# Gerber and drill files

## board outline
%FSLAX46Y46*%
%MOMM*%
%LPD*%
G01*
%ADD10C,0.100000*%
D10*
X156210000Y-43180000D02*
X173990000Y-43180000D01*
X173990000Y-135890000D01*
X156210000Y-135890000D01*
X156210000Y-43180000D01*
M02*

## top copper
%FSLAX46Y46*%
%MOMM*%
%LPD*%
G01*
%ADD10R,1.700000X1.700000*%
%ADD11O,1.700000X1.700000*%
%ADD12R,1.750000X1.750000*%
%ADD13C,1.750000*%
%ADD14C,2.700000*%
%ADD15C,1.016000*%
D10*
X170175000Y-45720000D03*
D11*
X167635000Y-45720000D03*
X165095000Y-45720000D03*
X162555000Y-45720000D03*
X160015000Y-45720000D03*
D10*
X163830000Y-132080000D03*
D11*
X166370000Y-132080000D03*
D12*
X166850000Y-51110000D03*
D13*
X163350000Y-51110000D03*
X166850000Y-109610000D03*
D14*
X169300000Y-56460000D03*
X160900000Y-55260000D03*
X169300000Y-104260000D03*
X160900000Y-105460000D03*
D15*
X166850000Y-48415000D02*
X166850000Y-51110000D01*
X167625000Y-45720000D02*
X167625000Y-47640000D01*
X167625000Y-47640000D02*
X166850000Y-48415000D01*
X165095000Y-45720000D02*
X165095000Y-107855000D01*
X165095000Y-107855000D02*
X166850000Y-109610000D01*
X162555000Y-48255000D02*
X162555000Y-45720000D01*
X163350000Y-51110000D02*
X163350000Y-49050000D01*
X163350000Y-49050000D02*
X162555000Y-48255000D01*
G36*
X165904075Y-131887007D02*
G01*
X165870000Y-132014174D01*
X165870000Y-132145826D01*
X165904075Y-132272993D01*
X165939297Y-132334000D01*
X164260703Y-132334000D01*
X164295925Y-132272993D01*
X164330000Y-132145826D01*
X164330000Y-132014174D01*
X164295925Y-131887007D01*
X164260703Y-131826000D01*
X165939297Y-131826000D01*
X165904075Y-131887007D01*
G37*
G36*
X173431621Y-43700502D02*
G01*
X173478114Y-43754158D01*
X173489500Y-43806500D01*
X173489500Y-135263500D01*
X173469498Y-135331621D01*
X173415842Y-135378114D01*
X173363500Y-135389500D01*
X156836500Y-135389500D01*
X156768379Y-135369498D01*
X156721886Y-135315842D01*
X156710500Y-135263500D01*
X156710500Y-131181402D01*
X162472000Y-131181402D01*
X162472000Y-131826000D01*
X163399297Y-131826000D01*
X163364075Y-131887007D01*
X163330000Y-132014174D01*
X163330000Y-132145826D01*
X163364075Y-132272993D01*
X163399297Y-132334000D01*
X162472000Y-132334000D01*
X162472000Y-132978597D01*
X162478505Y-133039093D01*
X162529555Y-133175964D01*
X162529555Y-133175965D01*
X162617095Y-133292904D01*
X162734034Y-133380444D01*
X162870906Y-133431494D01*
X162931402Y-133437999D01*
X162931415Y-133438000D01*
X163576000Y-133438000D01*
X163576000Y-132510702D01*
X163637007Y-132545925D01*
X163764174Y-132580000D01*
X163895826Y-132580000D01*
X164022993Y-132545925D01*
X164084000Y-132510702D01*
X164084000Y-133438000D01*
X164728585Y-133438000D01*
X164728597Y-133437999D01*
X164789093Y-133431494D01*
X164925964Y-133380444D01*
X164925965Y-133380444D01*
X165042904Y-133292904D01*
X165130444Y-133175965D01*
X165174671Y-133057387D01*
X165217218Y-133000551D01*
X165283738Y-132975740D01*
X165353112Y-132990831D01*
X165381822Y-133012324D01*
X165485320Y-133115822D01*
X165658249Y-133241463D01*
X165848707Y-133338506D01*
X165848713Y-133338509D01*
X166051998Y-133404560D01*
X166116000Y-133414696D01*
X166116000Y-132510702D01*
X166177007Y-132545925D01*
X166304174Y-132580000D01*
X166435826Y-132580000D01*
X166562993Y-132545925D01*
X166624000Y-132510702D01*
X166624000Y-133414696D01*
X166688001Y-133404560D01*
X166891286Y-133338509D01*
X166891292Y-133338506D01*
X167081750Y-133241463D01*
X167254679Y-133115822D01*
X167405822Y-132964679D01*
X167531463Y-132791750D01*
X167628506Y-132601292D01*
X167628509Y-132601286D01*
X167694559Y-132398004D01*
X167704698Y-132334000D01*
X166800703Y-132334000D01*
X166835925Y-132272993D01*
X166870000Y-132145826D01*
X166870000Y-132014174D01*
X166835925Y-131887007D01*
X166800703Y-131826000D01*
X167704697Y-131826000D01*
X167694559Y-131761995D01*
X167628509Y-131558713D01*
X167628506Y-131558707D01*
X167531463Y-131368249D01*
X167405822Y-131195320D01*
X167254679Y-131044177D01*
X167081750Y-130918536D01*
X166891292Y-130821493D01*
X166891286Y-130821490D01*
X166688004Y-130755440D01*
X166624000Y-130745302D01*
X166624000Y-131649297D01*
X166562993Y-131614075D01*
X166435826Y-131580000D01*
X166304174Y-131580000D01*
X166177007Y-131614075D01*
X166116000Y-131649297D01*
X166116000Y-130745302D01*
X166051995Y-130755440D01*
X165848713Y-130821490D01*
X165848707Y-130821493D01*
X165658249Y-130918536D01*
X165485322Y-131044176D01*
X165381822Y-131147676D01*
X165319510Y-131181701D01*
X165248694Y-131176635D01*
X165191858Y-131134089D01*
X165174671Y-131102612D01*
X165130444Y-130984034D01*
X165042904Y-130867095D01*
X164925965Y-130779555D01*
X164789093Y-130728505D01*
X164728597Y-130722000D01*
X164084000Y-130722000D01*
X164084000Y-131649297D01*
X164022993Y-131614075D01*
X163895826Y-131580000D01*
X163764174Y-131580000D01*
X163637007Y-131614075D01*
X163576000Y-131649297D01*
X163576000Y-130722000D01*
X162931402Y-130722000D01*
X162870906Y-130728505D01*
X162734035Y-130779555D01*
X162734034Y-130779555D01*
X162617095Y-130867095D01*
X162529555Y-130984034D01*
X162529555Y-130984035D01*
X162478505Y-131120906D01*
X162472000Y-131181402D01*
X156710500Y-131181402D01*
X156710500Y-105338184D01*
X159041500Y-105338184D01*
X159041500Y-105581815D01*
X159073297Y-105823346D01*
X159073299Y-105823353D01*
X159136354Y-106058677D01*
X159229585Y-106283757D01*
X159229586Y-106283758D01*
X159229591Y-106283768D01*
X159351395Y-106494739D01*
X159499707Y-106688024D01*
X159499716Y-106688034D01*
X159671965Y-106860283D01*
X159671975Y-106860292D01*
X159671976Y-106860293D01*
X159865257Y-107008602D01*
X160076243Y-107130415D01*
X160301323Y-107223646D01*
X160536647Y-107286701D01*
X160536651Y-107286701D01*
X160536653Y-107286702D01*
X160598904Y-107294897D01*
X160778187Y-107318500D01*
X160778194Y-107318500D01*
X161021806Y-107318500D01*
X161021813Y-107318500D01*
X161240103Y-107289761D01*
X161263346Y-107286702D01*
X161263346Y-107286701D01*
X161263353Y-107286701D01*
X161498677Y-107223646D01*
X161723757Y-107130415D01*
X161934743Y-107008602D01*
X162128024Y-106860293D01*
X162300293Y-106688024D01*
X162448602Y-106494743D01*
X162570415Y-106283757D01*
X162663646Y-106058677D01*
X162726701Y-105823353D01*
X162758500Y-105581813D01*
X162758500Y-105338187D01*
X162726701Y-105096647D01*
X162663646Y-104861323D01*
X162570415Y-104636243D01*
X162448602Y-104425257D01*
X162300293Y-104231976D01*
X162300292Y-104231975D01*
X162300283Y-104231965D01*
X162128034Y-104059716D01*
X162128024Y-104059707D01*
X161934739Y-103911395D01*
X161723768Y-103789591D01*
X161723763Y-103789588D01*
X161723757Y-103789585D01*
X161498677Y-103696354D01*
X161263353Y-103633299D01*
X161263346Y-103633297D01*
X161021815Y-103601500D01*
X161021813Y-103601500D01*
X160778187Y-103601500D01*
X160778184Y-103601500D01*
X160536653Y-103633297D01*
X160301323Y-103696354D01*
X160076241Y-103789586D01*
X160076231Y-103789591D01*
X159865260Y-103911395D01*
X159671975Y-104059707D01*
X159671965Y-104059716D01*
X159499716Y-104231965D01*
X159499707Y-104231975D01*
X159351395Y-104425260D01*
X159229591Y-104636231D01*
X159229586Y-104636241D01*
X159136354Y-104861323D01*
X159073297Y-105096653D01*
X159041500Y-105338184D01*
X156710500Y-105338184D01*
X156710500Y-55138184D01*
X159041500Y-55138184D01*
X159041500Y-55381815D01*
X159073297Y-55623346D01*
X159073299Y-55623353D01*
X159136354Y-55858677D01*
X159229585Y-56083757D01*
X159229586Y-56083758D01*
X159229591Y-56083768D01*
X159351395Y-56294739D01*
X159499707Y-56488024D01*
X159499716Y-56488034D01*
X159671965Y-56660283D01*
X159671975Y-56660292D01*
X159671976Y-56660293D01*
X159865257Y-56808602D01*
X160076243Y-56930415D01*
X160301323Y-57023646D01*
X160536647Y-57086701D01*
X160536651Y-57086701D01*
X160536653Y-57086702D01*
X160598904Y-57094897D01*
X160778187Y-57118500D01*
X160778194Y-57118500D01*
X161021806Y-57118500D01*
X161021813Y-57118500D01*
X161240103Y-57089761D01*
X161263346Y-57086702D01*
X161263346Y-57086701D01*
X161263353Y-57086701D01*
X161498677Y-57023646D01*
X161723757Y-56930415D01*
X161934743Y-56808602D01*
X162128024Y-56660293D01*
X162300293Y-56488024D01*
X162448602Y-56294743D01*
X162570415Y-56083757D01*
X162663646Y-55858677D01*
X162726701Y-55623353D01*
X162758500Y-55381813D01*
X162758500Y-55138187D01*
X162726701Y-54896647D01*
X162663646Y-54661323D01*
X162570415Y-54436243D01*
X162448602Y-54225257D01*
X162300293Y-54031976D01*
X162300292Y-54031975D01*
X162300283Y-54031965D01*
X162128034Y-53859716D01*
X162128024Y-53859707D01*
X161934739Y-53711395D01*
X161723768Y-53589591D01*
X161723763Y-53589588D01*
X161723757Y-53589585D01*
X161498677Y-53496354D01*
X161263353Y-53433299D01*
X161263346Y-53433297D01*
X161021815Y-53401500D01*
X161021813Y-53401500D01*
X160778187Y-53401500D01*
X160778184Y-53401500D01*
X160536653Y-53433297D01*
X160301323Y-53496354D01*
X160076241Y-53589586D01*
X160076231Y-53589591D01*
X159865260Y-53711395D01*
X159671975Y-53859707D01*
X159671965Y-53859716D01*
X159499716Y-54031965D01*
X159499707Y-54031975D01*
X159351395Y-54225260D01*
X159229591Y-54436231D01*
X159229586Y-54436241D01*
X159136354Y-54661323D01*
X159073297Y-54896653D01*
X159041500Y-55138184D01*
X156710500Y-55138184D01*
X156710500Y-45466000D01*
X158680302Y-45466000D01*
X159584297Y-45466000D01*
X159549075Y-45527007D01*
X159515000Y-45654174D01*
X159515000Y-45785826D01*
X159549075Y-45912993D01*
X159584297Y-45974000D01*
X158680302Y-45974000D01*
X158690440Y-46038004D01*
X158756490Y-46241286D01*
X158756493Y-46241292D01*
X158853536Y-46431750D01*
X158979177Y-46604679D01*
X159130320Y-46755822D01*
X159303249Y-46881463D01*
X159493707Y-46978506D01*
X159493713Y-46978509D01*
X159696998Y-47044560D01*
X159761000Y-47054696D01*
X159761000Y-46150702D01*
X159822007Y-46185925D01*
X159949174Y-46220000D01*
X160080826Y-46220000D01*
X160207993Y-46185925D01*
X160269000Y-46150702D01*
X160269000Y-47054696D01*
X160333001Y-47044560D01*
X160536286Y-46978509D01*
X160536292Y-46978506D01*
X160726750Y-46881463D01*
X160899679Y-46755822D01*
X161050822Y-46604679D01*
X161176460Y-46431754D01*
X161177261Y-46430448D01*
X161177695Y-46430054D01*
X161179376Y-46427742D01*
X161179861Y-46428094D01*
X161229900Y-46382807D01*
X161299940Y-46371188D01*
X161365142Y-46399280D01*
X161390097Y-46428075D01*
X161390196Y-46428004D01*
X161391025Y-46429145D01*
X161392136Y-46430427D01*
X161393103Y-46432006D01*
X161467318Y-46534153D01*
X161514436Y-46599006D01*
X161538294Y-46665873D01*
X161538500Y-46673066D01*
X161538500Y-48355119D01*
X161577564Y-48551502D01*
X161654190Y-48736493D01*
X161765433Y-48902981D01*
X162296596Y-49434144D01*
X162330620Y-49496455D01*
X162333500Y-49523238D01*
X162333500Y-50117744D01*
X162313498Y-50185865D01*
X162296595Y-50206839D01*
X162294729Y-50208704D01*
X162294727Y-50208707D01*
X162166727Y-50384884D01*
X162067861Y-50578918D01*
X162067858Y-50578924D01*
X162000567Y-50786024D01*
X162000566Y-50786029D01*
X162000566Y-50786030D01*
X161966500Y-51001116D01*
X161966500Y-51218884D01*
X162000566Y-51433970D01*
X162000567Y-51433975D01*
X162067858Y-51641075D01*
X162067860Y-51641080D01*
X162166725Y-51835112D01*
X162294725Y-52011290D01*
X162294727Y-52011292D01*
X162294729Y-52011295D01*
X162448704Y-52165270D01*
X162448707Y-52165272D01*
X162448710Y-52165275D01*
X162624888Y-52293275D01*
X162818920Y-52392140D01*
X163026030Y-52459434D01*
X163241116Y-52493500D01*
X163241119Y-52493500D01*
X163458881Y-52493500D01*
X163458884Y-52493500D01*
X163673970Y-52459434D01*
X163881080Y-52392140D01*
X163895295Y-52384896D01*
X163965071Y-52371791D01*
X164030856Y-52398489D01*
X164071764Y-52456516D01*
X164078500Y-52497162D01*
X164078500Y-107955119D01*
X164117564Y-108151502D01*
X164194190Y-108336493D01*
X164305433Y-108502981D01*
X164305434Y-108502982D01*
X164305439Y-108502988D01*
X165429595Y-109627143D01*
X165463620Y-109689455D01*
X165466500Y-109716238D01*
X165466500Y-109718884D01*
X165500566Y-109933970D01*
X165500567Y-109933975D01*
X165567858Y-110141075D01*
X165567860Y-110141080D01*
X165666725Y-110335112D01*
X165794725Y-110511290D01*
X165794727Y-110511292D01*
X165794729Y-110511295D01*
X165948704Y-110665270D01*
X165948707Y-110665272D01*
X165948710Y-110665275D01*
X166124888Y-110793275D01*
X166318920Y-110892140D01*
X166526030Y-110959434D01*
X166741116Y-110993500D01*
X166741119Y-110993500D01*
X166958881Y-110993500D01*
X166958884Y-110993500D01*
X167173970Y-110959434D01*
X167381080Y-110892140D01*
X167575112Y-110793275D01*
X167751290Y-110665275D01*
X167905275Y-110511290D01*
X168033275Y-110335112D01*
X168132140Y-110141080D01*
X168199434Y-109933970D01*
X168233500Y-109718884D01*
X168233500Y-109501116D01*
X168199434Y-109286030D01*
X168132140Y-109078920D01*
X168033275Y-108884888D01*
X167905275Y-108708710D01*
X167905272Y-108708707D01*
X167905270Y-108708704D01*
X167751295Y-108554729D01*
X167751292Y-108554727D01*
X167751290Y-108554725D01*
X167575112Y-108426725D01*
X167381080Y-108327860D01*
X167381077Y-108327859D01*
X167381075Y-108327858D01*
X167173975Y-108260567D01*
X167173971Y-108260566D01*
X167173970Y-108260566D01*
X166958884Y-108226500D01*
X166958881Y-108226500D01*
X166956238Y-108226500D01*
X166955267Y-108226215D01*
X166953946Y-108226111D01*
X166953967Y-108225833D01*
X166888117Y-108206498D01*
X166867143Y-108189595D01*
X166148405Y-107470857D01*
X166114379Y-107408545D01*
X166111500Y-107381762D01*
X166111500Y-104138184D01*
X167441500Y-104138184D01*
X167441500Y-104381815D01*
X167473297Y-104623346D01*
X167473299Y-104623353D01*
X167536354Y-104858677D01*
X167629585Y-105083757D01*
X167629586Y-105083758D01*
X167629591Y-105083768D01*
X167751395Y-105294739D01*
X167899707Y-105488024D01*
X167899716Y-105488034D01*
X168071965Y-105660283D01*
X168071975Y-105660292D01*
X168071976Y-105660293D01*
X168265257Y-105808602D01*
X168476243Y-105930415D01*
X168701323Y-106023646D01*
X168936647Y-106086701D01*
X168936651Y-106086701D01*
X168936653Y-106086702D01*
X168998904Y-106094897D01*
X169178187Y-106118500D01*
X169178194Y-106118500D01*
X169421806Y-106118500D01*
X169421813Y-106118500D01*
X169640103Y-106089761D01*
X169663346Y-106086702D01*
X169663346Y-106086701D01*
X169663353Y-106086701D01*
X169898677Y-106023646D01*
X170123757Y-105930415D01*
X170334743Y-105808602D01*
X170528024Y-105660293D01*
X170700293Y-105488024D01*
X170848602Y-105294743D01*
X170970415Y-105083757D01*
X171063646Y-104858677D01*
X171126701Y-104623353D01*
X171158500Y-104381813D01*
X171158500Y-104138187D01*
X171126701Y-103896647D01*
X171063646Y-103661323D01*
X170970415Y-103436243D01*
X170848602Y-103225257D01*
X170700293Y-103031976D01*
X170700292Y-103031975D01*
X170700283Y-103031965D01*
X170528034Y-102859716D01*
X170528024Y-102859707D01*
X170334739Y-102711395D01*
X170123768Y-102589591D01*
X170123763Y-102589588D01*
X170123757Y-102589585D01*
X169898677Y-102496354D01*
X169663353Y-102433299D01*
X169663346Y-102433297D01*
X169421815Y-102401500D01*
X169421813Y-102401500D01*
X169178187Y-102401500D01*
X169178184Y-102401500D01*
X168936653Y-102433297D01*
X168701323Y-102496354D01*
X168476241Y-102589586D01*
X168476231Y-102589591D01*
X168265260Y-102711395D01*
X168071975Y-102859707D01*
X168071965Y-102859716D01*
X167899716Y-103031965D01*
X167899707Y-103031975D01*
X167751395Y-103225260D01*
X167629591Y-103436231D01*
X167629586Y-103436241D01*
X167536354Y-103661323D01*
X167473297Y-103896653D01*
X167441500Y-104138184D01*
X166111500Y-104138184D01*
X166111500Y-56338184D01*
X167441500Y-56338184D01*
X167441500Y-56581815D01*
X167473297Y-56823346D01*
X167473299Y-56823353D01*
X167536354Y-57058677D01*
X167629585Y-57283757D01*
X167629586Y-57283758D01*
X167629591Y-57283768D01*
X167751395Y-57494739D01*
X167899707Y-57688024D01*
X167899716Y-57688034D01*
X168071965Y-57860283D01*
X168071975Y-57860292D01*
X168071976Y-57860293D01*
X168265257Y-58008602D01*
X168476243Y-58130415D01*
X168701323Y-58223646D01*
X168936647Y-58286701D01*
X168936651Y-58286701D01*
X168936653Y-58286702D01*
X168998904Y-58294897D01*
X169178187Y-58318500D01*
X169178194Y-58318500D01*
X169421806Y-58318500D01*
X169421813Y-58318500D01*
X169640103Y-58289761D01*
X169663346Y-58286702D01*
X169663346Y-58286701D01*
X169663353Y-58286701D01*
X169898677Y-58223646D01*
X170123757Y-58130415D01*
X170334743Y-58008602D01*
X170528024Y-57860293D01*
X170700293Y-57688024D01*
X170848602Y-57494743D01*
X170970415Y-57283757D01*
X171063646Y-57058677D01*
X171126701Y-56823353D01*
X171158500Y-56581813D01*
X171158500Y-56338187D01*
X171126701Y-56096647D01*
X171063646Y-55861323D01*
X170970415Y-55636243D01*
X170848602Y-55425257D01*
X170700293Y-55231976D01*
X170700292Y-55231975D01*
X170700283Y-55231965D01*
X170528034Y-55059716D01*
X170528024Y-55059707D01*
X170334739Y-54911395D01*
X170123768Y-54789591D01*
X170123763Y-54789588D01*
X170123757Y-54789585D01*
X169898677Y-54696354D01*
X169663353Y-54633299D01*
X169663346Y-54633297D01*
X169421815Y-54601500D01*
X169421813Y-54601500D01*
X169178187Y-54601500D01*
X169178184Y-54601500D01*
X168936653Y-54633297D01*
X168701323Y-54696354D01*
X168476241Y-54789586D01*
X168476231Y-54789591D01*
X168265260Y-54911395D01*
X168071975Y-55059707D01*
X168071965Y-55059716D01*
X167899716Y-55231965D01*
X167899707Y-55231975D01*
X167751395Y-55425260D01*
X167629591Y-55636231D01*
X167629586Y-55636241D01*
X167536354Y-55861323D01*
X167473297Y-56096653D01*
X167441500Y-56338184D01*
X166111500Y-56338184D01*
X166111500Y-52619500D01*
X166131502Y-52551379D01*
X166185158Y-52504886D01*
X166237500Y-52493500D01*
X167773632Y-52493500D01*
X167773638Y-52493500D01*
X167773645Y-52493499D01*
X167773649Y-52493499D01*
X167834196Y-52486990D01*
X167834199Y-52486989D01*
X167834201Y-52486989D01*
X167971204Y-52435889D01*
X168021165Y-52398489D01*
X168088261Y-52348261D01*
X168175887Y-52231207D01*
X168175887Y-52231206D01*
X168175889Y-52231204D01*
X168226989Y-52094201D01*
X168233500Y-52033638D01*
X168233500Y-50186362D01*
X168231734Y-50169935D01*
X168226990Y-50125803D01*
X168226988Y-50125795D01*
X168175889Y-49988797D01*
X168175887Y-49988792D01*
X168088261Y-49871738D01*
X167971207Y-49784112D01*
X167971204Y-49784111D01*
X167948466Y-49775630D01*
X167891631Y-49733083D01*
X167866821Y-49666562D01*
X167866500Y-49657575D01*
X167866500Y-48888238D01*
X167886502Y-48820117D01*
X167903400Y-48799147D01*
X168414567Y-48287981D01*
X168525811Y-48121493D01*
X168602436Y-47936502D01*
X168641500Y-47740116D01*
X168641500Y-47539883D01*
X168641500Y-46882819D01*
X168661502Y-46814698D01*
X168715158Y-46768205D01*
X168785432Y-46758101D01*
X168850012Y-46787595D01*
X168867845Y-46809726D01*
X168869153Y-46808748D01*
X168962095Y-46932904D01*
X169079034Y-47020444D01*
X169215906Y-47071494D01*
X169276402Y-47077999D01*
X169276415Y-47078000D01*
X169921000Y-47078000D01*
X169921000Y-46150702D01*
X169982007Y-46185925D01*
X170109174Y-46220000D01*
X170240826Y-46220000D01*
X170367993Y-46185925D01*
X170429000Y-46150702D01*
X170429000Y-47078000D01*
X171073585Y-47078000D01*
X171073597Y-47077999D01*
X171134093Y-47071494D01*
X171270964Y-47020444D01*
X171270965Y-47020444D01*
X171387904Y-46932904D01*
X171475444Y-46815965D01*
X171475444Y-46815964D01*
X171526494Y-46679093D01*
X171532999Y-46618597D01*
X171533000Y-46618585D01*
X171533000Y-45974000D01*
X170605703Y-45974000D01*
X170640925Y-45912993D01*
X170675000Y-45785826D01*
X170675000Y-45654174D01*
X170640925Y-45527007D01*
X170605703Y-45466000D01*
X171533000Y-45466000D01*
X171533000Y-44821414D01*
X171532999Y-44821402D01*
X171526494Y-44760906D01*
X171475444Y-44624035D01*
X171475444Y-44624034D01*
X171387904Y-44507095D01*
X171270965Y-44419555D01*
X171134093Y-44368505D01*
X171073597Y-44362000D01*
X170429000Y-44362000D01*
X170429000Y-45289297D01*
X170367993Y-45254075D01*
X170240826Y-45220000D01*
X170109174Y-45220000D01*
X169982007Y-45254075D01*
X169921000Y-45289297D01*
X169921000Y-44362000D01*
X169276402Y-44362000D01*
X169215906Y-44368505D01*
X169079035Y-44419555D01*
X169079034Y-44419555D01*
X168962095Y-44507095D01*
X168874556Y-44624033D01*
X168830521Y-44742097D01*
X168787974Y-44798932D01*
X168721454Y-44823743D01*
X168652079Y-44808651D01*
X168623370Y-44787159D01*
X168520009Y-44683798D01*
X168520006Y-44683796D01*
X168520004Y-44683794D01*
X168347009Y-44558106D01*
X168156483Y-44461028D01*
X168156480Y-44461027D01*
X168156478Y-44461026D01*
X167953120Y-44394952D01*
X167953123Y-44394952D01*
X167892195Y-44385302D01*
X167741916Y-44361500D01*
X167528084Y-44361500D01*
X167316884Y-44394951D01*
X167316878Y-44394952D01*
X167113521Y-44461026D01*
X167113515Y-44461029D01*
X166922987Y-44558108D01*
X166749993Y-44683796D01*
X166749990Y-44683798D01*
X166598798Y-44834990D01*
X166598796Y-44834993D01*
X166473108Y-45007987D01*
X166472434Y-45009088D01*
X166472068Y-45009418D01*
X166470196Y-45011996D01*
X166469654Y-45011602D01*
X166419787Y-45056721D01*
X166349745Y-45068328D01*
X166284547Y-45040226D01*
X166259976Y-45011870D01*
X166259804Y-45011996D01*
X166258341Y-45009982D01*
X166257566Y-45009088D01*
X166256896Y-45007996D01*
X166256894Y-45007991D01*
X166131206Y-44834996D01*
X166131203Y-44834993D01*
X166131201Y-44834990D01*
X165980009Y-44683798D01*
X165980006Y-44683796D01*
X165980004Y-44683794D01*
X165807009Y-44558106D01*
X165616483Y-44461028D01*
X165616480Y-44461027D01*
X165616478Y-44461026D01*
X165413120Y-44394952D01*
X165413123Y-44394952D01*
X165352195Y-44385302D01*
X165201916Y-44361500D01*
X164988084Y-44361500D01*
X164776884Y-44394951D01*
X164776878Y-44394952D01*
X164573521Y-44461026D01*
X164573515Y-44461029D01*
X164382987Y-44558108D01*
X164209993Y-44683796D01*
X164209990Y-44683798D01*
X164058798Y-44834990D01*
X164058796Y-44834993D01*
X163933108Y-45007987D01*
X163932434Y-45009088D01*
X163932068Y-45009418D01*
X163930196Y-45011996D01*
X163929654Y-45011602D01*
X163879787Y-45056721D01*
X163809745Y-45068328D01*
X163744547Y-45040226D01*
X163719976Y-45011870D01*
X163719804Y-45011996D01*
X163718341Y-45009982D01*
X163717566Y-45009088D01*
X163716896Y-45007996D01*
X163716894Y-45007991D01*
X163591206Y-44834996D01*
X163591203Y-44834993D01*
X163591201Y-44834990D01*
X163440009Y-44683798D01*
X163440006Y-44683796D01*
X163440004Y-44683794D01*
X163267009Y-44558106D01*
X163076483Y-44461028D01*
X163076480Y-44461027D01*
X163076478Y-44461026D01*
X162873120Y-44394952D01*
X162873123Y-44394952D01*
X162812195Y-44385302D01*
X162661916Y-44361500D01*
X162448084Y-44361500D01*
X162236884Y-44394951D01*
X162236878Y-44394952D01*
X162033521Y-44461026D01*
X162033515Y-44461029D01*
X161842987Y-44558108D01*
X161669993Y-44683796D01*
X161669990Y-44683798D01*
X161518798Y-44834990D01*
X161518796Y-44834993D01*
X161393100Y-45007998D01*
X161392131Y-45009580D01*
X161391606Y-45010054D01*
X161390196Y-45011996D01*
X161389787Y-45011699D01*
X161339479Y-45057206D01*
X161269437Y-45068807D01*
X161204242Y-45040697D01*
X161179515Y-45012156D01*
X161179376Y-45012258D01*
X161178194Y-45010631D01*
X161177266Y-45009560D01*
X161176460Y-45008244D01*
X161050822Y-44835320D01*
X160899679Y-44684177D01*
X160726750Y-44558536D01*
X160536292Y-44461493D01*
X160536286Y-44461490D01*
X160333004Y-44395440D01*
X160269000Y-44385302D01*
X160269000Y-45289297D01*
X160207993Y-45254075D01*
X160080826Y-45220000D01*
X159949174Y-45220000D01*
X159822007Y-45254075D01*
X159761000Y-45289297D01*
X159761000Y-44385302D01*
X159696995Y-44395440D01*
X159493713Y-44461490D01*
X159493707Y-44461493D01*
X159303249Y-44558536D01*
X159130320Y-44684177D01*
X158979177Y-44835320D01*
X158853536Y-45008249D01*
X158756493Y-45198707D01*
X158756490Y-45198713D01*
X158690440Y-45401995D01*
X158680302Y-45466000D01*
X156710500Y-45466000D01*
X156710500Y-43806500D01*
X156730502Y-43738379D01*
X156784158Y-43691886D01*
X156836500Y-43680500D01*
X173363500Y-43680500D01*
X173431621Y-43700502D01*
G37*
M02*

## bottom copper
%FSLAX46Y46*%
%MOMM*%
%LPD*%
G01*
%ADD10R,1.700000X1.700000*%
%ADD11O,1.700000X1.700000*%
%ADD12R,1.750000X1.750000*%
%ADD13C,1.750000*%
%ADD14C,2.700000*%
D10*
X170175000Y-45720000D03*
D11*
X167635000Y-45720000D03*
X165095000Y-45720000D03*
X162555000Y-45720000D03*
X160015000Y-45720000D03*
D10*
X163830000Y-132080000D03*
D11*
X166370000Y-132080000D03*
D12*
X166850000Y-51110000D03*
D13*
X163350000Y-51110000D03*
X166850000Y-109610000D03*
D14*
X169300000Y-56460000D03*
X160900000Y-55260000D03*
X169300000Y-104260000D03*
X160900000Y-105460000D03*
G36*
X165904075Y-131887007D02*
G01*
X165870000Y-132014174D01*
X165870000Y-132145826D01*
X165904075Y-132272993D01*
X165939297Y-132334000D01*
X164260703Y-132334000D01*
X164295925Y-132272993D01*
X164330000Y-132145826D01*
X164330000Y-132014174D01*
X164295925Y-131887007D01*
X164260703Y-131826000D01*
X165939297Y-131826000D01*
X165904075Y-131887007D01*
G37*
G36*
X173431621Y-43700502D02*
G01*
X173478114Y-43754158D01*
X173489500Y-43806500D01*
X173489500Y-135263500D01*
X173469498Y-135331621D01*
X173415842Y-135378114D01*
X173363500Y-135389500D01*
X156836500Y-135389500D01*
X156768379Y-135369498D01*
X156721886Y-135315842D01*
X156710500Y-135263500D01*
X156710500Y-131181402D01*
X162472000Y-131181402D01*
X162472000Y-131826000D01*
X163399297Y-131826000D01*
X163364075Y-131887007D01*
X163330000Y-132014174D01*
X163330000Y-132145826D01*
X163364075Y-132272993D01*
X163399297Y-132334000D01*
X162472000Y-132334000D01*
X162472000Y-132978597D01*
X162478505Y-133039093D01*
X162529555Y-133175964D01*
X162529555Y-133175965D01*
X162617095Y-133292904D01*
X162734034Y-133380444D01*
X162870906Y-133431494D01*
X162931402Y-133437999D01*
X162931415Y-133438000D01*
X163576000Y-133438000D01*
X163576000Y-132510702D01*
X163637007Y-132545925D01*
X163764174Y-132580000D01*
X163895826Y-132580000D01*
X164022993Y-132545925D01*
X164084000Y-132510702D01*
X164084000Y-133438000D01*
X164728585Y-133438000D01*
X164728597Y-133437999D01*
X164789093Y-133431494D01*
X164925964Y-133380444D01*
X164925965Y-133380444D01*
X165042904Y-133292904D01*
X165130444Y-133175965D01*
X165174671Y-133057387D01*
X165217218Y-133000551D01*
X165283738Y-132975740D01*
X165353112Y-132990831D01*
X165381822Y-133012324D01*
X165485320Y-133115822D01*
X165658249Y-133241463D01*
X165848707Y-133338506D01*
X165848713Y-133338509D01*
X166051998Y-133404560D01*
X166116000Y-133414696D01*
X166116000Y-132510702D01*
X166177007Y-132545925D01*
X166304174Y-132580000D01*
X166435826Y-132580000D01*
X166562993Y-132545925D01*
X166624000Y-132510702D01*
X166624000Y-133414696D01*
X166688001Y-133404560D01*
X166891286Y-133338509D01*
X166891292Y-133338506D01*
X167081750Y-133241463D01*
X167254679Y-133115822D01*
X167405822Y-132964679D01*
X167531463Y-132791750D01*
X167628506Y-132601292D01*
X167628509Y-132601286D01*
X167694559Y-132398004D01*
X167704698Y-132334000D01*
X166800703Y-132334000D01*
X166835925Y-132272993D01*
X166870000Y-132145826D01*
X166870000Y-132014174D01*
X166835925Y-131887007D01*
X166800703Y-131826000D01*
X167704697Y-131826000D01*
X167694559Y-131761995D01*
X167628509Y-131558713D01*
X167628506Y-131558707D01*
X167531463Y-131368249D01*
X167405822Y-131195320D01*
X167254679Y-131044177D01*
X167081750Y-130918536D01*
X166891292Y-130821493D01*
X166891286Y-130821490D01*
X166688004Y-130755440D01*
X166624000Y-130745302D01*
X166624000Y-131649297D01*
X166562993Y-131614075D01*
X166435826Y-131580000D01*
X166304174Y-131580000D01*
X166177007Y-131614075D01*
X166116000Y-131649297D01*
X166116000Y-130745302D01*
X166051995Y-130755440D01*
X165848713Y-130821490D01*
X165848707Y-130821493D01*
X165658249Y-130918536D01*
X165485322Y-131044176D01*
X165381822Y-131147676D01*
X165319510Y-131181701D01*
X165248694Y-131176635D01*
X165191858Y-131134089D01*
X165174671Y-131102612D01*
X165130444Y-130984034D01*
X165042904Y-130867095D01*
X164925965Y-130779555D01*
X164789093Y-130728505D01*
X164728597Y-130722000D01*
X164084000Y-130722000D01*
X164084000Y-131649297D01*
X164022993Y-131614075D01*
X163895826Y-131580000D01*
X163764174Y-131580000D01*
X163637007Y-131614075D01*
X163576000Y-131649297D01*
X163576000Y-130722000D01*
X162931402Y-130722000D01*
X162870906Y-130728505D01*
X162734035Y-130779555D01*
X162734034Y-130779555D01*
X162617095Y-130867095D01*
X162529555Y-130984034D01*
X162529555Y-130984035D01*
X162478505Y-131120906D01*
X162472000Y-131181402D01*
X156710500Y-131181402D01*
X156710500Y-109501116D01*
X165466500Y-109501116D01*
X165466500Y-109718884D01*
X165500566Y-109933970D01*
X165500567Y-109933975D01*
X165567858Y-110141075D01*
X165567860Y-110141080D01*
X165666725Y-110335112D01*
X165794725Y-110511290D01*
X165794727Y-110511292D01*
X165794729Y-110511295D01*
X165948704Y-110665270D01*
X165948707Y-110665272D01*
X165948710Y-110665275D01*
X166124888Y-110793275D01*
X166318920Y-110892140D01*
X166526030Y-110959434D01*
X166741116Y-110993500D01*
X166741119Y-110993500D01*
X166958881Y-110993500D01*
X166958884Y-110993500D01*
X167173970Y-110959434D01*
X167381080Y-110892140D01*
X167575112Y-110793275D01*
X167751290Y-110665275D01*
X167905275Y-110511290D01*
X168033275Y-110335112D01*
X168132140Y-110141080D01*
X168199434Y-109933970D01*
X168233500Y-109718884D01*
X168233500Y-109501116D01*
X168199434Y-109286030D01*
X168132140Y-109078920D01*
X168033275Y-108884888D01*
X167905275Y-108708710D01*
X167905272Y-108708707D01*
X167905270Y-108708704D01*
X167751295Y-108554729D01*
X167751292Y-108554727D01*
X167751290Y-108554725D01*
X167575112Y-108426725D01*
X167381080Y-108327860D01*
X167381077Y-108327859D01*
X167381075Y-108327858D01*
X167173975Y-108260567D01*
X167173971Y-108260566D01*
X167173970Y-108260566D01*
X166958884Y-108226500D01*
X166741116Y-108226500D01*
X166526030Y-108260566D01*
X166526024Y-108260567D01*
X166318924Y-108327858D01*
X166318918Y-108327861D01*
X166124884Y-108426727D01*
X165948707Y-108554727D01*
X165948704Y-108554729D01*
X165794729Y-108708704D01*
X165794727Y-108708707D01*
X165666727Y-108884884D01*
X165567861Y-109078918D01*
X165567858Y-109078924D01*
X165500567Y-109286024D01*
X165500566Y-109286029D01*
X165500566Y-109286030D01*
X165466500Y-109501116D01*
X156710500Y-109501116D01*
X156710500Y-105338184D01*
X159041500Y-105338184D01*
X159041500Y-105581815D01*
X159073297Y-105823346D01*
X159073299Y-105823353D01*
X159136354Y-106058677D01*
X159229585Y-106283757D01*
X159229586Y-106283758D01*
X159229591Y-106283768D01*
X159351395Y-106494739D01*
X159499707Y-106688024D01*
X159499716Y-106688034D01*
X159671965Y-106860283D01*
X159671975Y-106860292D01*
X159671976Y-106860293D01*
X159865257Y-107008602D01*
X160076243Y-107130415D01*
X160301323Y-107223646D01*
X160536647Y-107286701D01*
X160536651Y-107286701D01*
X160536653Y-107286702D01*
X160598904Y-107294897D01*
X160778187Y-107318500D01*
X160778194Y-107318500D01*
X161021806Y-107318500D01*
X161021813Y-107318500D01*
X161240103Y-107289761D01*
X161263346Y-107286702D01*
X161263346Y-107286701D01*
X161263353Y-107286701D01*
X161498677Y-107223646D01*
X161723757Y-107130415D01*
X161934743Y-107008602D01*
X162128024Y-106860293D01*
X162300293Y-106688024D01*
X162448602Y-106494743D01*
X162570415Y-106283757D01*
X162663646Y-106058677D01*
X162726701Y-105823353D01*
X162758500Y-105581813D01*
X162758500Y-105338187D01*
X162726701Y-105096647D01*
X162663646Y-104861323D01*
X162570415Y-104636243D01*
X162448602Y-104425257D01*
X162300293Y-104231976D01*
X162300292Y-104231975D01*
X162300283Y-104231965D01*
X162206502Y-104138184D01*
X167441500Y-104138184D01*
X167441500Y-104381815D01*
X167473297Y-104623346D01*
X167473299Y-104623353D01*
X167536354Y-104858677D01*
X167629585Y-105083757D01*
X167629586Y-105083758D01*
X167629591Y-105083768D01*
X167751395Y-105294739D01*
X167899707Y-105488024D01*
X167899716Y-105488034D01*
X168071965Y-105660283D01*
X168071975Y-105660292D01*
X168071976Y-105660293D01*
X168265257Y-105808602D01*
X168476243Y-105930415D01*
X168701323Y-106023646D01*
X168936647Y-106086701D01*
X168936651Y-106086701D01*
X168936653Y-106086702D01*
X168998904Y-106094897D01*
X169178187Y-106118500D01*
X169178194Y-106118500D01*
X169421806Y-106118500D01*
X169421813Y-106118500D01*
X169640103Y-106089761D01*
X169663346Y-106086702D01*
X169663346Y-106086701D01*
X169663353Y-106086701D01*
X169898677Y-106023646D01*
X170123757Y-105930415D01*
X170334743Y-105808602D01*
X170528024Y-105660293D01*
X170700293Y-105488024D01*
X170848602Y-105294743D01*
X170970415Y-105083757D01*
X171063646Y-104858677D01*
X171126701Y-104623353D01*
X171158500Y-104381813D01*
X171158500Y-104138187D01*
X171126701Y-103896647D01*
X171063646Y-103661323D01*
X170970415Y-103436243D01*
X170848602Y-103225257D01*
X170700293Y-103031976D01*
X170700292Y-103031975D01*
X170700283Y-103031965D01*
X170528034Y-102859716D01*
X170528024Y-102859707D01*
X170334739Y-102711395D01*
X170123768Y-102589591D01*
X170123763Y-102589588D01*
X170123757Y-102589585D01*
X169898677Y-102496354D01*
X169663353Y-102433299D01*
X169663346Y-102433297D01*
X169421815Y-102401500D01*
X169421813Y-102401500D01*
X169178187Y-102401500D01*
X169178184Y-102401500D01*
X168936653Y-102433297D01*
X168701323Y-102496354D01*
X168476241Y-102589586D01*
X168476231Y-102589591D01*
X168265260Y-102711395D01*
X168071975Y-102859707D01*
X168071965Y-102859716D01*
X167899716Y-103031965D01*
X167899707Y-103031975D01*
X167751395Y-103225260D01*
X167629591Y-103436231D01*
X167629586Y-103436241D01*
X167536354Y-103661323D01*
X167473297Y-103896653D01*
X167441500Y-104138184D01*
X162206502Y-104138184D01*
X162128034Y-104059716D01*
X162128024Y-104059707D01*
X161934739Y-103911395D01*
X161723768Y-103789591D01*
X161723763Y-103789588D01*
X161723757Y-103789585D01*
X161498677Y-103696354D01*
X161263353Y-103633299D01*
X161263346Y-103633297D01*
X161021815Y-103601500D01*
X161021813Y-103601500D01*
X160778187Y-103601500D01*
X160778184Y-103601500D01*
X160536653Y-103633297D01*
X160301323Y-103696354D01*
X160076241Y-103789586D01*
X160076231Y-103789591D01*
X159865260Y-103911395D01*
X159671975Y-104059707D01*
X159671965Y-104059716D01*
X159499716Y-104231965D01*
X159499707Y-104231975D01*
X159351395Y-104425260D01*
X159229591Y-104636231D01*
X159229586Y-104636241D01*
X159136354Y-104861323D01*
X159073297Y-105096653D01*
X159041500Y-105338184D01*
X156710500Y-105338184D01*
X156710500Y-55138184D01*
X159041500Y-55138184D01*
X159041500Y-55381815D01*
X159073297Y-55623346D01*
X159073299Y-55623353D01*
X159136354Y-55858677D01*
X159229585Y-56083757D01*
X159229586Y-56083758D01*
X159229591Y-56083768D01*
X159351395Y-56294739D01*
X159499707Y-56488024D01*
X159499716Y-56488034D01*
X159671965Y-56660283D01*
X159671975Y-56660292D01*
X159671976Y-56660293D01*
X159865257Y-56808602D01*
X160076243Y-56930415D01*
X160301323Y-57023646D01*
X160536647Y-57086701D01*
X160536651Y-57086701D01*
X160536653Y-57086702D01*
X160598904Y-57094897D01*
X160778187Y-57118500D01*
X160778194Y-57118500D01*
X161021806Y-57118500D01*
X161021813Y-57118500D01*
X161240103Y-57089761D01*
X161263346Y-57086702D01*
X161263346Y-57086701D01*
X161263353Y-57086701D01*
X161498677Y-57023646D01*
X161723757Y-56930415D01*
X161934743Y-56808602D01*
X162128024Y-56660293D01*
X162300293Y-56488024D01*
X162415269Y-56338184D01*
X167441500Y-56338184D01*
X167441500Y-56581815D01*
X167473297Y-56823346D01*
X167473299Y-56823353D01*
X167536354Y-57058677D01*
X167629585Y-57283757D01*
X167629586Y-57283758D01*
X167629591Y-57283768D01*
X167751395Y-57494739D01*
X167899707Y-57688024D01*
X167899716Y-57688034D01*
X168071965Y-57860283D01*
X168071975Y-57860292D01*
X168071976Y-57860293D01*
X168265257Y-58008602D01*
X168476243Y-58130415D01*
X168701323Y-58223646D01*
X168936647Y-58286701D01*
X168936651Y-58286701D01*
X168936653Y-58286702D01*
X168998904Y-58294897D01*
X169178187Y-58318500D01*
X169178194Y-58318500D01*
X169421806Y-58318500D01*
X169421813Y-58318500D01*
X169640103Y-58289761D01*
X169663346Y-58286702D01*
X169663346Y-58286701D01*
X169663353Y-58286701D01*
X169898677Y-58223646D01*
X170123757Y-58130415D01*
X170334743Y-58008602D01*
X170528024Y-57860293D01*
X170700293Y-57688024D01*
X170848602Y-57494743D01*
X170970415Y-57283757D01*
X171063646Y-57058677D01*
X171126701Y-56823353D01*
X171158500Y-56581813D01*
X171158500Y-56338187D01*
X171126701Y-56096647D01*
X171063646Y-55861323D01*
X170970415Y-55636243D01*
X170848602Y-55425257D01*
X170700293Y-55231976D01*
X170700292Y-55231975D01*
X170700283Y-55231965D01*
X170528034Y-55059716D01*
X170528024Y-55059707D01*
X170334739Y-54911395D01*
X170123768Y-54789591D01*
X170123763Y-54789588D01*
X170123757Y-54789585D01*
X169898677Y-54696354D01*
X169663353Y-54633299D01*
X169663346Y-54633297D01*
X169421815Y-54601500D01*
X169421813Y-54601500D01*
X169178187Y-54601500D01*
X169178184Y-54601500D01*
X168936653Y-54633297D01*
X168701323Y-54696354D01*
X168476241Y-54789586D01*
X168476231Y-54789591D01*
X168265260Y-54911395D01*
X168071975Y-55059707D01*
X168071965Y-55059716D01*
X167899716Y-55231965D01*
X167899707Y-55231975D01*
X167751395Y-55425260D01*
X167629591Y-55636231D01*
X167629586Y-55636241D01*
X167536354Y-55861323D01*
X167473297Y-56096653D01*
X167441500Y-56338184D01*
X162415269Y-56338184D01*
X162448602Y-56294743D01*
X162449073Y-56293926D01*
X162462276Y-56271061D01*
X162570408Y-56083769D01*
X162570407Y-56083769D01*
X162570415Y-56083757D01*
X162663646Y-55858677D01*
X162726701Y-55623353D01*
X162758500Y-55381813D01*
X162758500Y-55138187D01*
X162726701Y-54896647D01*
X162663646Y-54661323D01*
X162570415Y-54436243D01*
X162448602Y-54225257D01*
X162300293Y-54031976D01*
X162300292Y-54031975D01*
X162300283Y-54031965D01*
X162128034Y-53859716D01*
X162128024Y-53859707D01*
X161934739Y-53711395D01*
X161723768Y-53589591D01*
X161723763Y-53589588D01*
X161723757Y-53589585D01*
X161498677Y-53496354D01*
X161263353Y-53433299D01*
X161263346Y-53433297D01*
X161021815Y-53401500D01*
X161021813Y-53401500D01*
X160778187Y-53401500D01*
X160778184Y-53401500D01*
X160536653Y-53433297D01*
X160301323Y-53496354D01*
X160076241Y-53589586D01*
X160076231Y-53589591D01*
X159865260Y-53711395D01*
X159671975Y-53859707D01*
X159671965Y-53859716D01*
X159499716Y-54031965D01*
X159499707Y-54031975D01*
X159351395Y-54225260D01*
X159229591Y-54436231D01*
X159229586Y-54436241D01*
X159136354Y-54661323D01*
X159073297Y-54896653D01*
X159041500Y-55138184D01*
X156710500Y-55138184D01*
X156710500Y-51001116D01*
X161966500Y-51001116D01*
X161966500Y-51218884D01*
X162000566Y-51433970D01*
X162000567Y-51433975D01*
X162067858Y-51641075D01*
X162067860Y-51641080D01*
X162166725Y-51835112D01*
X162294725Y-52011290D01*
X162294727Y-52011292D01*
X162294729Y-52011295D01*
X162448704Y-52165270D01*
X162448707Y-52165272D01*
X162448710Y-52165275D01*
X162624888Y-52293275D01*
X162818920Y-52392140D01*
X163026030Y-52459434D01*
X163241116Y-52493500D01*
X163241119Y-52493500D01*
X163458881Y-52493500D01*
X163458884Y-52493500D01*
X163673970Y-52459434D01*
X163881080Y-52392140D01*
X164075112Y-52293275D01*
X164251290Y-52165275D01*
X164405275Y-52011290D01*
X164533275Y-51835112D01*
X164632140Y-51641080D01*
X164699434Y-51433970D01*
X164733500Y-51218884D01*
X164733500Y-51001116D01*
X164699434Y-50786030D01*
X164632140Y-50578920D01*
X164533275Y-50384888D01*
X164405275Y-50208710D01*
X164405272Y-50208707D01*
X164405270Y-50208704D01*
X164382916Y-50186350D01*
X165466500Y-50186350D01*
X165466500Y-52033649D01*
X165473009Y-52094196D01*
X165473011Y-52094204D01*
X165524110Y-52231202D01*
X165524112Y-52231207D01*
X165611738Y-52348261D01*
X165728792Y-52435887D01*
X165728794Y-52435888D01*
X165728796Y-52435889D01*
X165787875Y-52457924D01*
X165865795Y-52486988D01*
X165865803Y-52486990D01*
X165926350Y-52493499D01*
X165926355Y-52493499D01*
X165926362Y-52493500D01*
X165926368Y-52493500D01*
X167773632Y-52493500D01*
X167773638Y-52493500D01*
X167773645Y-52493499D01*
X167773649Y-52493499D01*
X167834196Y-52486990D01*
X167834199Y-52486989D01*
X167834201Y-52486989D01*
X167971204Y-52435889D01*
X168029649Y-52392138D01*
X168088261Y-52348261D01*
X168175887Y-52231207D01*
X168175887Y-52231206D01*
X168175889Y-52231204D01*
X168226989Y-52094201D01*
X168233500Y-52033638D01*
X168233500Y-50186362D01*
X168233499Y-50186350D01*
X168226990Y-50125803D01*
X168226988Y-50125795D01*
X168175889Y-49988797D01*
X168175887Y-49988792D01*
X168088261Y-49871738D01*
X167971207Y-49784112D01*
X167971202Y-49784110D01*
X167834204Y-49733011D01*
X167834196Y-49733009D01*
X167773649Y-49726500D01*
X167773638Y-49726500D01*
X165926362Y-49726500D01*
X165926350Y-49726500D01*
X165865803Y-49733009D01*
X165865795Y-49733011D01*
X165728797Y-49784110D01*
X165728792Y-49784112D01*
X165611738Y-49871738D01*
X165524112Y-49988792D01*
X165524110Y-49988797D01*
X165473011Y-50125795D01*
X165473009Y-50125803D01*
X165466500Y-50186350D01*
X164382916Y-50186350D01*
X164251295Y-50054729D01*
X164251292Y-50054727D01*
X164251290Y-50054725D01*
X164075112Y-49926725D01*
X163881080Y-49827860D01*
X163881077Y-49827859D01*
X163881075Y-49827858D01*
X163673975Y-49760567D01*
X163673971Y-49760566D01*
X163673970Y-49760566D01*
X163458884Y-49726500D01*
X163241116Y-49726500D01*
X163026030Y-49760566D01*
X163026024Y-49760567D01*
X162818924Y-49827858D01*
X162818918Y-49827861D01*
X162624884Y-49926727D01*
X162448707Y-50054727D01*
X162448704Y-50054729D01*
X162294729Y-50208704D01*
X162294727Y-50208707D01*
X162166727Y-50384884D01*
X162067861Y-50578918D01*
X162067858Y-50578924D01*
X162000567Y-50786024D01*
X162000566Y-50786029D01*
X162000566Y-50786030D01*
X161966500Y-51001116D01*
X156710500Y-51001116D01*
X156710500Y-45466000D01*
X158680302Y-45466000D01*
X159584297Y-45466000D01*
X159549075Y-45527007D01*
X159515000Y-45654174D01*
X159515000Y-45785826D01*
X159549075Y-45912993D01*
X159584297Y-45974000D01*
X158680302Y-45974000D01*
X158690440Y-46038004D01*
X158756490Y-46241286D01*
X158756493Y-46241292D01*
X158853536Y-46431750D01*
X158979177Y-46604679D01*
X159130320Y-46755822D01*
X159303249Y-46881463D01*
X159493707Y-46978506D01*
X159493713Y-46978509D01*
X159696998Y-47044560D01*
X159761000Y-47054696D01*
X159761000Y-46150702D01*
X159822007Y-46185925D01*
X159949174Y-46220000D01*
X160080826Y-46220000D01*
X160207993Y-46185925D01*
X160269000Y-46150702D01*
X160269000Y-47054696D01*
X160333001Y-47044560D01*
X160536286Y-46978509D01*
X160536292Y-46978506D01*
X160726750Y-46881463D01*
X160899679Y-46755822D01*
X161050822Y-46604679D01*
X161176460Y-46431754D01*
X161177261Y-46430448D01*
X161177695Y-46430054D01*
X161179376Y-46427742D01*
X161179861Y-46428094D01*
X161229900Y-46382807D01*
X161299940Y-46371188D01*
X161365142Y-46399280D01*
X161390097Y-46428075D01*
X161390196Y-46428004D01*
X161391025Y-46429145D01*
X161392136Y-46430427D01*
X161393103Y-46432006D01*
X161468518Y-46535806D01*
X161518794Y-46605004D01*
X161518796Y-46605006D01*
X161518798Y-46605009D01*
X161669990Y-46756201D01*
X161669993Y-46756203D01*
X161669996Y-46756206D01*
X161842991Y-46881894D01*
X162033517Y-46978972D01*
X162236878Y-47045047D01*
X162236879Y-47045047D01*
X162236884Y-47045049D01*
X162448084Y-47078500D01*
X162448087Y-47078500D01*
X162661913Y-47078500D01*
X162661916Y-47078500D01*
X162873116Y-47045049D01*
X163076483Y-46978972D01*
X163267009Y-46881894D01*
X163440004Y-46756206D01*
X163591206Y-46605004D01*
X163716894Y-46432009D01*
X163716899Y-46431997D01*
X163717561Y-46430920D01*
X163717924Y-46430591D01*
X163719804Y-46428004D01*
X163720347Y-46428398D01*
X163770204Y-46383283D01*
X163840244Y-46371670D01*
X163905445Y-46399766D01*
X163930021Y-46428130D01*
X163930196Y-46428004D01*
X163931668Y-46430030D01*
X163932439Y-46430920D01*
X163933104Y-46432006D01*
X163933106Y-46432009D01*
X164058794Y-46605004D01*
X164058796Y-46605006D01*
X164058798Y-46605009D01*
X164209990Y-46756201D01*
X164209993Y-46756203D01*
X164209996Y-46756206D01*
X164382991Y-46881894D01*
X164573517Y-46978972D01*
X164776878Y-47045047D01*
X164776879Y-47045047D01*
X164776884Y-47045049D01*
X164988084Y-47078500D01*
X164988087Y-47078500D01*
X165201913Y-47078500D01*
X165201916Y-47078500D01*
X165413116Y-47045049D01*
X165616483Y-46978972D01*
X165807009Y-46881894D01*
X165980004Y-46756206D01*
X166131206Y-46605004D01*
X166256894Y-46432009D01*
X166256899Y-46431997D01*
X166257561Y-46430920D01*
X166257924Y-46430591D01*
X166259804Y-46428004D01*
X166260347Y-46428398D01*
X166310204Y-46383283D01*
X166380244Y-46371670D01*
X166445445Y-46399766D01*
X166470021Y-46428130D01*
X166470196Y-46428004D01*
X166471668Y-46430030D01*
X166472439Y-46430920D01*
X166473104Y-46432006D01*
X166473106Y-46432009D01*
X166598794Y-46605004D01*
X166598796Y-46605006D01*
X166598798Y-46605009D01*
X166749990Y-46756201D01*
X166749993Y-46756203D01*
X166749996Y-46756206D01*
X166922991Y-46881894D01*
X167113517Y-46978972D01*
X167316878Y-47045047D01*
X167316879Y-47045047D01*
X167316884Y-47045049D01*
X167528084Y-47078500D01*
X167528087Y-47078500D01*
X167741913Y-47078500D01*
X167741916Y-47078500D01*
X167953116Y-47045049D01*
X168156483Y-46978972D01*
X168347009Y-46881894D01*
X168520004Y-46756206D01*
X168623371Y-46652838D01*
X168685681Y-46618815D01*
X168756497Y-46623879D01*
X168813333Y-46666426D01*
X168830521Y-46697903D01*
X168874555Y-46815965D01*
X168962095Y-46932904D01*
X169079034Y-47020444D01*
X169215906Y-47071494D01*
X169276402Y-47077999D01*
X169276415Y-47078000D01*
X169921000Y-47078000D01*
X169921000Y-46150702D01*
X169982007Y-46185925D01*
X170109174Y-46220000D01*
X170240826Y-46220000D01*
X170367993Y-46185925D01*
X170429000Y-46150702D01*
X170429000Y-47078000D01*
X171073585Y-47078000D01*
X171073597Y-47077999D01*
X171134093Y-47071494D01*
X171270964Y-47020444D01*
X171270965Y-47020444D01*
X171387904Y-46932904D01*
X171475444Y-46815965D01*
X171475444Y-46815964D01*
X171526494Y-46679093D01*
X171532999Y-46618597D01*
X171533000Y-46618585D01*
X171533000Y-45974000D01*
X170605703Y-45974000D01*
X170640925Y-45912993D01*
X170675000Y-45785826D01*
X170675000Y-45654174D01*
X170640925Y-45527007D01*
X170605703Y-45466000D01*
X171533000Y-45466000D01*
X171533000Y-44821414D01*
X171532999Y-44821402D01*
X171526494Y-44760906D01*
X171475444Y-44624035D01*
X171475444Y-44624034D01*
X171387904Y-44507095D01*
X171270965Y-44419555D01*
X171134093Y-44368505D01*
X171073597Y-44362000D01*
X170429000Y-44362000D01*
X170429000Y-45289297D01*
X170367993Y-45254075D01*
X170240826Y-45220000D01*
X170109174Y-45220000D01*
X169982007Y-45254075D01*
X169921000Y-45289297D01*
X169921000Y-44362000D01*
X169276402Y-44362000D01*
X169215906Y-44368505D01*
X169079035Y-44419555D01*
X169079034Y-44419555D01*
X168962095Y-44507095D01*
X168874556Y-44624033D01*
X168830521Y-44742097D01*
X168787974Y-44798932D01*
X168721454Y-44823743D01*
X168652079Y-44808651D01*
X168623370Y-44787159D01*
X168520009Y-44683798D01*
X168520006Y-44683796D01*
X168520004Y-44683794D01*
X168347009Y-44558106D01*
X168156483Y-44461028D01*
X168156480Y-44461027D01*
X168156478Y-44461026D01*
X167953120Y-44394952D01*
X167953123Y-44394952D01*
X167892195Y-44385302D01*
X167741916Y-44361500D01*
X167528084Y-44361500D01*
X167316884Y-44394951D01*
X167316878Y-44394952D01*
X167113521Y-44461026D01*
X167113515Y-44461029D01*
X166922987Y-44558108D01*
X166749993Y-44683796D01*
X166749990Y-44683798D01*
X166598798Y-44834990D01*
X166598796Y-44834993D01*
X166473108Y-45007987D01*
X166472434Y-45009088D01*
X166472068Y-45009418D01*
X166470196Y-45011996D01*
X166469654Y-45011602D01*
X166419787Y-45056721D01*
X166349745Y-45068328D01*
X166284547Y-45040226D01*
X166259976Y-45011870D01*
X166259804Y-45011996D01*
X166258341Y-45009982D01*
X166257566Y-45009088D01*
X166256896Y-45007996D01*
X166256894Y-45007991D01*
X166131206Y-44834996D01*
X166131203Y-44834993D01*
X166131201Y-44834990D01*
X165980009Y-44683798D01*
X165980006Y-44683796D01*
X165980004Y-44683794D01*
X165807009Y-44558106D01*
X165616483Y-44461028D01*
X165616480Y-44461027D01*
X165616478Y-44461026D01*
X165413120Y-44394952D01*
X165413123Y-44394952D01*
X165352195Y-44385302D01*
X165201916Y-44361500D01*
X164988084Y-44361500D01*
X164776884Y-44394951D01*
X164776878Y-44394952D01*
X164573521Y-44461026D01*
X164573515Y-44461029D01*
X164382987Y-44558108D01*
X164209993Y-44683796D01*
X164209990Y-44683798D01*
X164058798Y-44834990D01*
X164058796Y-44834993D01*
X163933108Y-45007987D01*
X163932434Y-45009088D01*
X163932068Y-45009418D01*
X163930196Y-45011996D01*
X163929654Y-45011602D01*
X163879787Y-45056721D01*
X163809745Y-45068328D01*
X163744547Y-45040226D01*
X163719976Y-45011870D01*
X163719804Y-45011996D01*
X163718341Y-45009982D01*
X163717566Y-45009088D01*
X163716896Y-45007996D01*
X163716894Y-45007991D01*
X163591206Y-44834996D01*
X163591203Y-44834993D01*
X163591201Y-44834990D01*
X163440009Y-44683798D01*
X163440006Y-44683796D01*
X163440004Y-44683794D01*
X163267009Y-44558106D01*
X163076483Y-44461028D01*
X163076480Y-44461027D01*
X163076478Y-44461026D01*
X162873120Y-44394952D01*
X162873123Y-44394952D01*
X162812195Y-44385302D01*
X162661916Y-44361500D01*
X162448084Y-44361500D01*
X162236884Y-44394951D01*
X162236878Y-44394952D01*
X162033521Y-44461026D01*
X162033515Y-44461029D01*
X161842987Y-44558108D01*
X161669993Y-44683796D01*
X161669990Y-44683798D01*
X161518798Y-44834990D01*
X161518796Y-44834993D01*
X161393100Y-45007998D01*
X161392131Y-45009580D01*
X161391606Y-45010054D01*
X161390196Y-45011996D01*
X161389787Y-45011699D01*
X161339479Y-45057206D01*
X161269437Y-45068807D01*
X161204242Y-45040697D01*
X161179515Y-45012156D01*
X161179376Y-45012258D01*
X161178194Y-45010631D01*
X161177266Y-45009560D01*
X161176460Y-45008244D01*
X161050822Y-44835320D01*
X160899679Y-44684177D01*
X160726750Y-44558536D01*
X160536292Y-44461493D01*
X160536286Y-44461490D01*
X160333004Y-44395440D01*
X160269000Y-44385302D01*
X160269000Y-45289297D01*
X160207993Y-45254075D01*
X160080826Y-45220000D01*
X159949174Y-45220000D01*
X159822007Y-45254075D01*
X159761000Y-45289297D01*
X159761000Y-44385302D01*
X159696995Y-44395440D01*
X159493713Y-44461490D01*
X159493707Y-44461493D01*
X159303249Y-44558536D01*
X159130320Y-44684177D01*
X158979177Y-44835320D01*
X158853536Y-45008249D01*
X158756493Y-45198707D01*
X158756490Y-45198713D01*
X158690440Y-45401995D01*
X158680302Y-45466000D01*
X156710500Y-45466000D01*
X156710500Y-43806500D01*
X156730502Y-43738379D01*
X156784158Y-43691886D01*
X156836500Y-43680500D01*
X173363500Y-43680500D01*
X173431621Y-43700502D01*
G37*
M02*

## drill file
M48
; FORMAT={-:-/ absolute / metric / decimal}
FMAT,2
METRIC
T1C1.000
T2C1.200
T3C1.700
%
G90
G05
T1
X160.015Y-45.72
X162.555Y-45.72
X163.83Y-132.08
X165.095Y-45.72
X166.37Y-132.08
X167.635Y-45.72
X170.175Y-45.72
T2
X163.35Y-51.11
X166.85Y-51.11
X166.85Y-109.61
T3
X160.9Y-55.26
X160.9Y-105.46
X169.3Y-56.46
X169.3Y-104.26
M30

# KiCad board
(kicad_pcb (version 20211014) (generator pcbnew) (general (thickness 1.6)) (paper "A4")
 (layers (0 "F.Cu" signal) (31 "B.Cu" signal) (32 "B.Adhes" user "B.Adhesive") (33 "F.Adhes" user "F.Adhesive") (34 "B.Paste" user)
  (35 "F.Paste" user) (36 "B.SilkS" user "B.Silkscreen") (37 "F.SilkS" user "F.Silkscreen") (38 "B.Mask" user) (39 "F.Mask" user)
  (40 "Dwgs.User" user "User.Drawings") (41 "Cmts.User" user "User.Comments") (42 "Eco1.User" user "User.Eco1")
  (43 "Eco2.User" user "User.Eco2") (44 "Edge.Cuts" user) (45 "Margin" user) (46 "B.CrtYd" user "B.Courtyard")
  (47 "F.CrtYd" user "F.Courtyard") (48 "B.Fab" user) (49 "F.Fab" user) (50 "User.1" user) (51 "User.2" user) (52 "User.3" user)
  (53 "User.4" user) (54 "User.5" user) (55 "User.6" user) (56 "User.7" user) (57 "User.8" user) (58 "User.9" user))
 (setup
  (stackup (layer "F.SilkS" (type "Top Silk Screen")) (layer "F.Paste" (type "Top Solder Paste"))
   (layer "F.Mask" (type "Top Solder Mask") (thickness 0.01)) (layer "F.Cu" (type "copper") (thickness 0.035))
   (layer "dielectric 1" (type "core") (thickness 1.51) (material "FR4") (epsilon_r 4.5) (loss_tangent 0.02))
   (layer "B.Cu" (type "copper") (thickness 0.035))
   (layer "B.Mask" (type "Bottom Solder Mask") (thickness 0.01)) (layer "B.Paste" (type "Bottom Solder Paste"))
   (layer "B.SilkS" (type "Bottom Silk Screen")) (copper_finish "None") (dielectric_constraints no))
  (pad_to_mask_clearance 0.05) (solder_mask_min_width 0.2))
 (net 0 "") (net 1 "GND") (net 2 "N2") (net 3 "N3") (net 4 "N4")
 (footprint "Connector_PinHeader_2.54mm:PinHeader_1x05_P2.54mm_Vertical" (layer "F.Cu") (at 170.175 45.72 -90)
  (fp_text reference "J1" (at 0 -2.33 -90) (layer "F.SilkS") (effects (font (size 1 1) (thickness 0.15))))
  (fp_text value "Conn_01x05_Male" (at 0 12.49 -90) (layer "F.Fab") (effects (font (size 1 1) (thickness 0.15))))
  (pad "1" thru_hole rect (at 0 0 270) (size 1.7 1.7) (drill 1) (layers *.Cu *.Mask) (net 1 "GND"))
  (pad "2" thru_hole oval (at 0 2.54 270) (size 1.7 1.7) (drill 1) (layers *.Cu *.Mask) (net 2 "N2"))
  (pad "3" thru_hole oval (at 0 5.08 270) (size 1.7 1.7) (drill 1) (layers *.Cu *.Mask) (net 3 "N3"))
  (pad "4" thru_hole oval (at 0 7.62 270) (size 1.7 1.7) (drill 1) (layers *.Cu *.Mask) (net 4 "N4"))
  (pad "5" thru_hole oval (at 0 10.16 270) (size 1.7 1.7) (drill 1) (layers *.Cu *.Mask) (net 1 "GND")))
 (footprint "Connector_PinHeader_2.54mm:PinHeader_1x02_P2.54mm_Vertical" (layer "F.Cu") (at 163.83 132.08 90)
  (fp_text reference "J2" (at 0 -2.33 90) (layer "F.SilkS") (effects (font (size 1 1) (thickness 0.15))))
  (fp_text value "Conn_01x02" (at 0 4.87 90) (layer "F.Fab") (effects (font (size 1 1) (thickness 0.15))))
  (pad "1" thru_hole rect (at 0 0 90) (size 1.7 1.7) (drill 1) (layers *.Cu *.Mask) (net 1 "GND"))
  (pad "2" thru_hole oval (at 0 2.54 90) (size 1.7 1.7) (drill 1) (layers *.Cu *.Mask) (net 1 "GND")))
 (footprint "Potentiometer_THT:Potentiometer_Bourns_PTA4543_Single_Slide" (layer "F.Cu") (at 166.85 51.11 -90)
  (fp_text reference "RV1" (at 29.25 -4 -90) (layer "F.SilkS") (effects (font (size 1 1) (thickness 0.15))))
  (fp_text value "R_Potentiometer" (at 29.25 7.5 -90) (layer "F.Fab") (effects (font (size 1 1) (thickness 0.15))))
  (pad "1" thru_hole rect (at 0 0 270) (size 1.75 1.75) (drill 1.2) (layers *.Cu *.Mask) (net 2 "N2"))
  (pad "2" thru_hole circle (at 0 3.5 270) (size 1.75 1.75) (drill 1.2) (layers *.Cu *.Mask) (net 4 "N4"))
  (pad "3" thru_hole circle (at 58.5 0 270) (size 1.75 1.75) (drill 1.2) (layers *.Cu *.Mask) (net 3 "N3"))
  (pad "MP" thru_hole circle (at 5.35 -2.45 270) (size 2.7 2.7) (drill 1.7) (layers *.Cu *.Mask))
  (pad "MP" thru_hole circle (at 4.15 5.95 270) (size 2.7 2.7) (drill 1.7) (layers *.Cu *.Mask))
  (pad "MP" thru_hole circle (at 53.15 -2.45 270) (size 2.7 2.7) (drill 1.7) (layers *.Cu *.Mask))
  (pad "MP" thru_hole circle (at 54.35 5.95 270) (size 2.7 2.7) (drill 1.7) (layers *.Cu *.Mask)))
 (gr_rect (start 156.21 43.18) (end 173.99 135.89) (layer "Edge.Cuts") (width 0.1) (fill none))
 (segment (start 166.85 48.415) (end 166.85 51.11) (width 1.016) (layer "F.Cu") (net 2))
 (segment (start 167.625 45.72) (end 167.625 47.64) (width 1.016) (layer "F.Cu") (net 2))
 (segment (start 167.625 47.64) (end 166.85 48.415) (width 1.016) (layer "F.Cu") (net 2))
 (segment (start 165.095 45.72) (end 165.095 107.855) (width 1.016) (layer "F.Cu") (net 3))
 (segment (start 165.095 107.855) (end 166.85 109.61) (width 1.016) (layer "F.Cu") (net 3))
 (segment (start 162.555 48.255) (end 162.555 45.72) (width 1.016) (layer "F.Cu") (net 4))
 (segment (start 163.35 51.11) (end 163.35 49.05) (width 1.016) (layer "F.Cu") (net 4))
 (segment (start 163.35 49.05) (end 162.555 48.255) (width 1.016) (layer "F.Cu") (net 4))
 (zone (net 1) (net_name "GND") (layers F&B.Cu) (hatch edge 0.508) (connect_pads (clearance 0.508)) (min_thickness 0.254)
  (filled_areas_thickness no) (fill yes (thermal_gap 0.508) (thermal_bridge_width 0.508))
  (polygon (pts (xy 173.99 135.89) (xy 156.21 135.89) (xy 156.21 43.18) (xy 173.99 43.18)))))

